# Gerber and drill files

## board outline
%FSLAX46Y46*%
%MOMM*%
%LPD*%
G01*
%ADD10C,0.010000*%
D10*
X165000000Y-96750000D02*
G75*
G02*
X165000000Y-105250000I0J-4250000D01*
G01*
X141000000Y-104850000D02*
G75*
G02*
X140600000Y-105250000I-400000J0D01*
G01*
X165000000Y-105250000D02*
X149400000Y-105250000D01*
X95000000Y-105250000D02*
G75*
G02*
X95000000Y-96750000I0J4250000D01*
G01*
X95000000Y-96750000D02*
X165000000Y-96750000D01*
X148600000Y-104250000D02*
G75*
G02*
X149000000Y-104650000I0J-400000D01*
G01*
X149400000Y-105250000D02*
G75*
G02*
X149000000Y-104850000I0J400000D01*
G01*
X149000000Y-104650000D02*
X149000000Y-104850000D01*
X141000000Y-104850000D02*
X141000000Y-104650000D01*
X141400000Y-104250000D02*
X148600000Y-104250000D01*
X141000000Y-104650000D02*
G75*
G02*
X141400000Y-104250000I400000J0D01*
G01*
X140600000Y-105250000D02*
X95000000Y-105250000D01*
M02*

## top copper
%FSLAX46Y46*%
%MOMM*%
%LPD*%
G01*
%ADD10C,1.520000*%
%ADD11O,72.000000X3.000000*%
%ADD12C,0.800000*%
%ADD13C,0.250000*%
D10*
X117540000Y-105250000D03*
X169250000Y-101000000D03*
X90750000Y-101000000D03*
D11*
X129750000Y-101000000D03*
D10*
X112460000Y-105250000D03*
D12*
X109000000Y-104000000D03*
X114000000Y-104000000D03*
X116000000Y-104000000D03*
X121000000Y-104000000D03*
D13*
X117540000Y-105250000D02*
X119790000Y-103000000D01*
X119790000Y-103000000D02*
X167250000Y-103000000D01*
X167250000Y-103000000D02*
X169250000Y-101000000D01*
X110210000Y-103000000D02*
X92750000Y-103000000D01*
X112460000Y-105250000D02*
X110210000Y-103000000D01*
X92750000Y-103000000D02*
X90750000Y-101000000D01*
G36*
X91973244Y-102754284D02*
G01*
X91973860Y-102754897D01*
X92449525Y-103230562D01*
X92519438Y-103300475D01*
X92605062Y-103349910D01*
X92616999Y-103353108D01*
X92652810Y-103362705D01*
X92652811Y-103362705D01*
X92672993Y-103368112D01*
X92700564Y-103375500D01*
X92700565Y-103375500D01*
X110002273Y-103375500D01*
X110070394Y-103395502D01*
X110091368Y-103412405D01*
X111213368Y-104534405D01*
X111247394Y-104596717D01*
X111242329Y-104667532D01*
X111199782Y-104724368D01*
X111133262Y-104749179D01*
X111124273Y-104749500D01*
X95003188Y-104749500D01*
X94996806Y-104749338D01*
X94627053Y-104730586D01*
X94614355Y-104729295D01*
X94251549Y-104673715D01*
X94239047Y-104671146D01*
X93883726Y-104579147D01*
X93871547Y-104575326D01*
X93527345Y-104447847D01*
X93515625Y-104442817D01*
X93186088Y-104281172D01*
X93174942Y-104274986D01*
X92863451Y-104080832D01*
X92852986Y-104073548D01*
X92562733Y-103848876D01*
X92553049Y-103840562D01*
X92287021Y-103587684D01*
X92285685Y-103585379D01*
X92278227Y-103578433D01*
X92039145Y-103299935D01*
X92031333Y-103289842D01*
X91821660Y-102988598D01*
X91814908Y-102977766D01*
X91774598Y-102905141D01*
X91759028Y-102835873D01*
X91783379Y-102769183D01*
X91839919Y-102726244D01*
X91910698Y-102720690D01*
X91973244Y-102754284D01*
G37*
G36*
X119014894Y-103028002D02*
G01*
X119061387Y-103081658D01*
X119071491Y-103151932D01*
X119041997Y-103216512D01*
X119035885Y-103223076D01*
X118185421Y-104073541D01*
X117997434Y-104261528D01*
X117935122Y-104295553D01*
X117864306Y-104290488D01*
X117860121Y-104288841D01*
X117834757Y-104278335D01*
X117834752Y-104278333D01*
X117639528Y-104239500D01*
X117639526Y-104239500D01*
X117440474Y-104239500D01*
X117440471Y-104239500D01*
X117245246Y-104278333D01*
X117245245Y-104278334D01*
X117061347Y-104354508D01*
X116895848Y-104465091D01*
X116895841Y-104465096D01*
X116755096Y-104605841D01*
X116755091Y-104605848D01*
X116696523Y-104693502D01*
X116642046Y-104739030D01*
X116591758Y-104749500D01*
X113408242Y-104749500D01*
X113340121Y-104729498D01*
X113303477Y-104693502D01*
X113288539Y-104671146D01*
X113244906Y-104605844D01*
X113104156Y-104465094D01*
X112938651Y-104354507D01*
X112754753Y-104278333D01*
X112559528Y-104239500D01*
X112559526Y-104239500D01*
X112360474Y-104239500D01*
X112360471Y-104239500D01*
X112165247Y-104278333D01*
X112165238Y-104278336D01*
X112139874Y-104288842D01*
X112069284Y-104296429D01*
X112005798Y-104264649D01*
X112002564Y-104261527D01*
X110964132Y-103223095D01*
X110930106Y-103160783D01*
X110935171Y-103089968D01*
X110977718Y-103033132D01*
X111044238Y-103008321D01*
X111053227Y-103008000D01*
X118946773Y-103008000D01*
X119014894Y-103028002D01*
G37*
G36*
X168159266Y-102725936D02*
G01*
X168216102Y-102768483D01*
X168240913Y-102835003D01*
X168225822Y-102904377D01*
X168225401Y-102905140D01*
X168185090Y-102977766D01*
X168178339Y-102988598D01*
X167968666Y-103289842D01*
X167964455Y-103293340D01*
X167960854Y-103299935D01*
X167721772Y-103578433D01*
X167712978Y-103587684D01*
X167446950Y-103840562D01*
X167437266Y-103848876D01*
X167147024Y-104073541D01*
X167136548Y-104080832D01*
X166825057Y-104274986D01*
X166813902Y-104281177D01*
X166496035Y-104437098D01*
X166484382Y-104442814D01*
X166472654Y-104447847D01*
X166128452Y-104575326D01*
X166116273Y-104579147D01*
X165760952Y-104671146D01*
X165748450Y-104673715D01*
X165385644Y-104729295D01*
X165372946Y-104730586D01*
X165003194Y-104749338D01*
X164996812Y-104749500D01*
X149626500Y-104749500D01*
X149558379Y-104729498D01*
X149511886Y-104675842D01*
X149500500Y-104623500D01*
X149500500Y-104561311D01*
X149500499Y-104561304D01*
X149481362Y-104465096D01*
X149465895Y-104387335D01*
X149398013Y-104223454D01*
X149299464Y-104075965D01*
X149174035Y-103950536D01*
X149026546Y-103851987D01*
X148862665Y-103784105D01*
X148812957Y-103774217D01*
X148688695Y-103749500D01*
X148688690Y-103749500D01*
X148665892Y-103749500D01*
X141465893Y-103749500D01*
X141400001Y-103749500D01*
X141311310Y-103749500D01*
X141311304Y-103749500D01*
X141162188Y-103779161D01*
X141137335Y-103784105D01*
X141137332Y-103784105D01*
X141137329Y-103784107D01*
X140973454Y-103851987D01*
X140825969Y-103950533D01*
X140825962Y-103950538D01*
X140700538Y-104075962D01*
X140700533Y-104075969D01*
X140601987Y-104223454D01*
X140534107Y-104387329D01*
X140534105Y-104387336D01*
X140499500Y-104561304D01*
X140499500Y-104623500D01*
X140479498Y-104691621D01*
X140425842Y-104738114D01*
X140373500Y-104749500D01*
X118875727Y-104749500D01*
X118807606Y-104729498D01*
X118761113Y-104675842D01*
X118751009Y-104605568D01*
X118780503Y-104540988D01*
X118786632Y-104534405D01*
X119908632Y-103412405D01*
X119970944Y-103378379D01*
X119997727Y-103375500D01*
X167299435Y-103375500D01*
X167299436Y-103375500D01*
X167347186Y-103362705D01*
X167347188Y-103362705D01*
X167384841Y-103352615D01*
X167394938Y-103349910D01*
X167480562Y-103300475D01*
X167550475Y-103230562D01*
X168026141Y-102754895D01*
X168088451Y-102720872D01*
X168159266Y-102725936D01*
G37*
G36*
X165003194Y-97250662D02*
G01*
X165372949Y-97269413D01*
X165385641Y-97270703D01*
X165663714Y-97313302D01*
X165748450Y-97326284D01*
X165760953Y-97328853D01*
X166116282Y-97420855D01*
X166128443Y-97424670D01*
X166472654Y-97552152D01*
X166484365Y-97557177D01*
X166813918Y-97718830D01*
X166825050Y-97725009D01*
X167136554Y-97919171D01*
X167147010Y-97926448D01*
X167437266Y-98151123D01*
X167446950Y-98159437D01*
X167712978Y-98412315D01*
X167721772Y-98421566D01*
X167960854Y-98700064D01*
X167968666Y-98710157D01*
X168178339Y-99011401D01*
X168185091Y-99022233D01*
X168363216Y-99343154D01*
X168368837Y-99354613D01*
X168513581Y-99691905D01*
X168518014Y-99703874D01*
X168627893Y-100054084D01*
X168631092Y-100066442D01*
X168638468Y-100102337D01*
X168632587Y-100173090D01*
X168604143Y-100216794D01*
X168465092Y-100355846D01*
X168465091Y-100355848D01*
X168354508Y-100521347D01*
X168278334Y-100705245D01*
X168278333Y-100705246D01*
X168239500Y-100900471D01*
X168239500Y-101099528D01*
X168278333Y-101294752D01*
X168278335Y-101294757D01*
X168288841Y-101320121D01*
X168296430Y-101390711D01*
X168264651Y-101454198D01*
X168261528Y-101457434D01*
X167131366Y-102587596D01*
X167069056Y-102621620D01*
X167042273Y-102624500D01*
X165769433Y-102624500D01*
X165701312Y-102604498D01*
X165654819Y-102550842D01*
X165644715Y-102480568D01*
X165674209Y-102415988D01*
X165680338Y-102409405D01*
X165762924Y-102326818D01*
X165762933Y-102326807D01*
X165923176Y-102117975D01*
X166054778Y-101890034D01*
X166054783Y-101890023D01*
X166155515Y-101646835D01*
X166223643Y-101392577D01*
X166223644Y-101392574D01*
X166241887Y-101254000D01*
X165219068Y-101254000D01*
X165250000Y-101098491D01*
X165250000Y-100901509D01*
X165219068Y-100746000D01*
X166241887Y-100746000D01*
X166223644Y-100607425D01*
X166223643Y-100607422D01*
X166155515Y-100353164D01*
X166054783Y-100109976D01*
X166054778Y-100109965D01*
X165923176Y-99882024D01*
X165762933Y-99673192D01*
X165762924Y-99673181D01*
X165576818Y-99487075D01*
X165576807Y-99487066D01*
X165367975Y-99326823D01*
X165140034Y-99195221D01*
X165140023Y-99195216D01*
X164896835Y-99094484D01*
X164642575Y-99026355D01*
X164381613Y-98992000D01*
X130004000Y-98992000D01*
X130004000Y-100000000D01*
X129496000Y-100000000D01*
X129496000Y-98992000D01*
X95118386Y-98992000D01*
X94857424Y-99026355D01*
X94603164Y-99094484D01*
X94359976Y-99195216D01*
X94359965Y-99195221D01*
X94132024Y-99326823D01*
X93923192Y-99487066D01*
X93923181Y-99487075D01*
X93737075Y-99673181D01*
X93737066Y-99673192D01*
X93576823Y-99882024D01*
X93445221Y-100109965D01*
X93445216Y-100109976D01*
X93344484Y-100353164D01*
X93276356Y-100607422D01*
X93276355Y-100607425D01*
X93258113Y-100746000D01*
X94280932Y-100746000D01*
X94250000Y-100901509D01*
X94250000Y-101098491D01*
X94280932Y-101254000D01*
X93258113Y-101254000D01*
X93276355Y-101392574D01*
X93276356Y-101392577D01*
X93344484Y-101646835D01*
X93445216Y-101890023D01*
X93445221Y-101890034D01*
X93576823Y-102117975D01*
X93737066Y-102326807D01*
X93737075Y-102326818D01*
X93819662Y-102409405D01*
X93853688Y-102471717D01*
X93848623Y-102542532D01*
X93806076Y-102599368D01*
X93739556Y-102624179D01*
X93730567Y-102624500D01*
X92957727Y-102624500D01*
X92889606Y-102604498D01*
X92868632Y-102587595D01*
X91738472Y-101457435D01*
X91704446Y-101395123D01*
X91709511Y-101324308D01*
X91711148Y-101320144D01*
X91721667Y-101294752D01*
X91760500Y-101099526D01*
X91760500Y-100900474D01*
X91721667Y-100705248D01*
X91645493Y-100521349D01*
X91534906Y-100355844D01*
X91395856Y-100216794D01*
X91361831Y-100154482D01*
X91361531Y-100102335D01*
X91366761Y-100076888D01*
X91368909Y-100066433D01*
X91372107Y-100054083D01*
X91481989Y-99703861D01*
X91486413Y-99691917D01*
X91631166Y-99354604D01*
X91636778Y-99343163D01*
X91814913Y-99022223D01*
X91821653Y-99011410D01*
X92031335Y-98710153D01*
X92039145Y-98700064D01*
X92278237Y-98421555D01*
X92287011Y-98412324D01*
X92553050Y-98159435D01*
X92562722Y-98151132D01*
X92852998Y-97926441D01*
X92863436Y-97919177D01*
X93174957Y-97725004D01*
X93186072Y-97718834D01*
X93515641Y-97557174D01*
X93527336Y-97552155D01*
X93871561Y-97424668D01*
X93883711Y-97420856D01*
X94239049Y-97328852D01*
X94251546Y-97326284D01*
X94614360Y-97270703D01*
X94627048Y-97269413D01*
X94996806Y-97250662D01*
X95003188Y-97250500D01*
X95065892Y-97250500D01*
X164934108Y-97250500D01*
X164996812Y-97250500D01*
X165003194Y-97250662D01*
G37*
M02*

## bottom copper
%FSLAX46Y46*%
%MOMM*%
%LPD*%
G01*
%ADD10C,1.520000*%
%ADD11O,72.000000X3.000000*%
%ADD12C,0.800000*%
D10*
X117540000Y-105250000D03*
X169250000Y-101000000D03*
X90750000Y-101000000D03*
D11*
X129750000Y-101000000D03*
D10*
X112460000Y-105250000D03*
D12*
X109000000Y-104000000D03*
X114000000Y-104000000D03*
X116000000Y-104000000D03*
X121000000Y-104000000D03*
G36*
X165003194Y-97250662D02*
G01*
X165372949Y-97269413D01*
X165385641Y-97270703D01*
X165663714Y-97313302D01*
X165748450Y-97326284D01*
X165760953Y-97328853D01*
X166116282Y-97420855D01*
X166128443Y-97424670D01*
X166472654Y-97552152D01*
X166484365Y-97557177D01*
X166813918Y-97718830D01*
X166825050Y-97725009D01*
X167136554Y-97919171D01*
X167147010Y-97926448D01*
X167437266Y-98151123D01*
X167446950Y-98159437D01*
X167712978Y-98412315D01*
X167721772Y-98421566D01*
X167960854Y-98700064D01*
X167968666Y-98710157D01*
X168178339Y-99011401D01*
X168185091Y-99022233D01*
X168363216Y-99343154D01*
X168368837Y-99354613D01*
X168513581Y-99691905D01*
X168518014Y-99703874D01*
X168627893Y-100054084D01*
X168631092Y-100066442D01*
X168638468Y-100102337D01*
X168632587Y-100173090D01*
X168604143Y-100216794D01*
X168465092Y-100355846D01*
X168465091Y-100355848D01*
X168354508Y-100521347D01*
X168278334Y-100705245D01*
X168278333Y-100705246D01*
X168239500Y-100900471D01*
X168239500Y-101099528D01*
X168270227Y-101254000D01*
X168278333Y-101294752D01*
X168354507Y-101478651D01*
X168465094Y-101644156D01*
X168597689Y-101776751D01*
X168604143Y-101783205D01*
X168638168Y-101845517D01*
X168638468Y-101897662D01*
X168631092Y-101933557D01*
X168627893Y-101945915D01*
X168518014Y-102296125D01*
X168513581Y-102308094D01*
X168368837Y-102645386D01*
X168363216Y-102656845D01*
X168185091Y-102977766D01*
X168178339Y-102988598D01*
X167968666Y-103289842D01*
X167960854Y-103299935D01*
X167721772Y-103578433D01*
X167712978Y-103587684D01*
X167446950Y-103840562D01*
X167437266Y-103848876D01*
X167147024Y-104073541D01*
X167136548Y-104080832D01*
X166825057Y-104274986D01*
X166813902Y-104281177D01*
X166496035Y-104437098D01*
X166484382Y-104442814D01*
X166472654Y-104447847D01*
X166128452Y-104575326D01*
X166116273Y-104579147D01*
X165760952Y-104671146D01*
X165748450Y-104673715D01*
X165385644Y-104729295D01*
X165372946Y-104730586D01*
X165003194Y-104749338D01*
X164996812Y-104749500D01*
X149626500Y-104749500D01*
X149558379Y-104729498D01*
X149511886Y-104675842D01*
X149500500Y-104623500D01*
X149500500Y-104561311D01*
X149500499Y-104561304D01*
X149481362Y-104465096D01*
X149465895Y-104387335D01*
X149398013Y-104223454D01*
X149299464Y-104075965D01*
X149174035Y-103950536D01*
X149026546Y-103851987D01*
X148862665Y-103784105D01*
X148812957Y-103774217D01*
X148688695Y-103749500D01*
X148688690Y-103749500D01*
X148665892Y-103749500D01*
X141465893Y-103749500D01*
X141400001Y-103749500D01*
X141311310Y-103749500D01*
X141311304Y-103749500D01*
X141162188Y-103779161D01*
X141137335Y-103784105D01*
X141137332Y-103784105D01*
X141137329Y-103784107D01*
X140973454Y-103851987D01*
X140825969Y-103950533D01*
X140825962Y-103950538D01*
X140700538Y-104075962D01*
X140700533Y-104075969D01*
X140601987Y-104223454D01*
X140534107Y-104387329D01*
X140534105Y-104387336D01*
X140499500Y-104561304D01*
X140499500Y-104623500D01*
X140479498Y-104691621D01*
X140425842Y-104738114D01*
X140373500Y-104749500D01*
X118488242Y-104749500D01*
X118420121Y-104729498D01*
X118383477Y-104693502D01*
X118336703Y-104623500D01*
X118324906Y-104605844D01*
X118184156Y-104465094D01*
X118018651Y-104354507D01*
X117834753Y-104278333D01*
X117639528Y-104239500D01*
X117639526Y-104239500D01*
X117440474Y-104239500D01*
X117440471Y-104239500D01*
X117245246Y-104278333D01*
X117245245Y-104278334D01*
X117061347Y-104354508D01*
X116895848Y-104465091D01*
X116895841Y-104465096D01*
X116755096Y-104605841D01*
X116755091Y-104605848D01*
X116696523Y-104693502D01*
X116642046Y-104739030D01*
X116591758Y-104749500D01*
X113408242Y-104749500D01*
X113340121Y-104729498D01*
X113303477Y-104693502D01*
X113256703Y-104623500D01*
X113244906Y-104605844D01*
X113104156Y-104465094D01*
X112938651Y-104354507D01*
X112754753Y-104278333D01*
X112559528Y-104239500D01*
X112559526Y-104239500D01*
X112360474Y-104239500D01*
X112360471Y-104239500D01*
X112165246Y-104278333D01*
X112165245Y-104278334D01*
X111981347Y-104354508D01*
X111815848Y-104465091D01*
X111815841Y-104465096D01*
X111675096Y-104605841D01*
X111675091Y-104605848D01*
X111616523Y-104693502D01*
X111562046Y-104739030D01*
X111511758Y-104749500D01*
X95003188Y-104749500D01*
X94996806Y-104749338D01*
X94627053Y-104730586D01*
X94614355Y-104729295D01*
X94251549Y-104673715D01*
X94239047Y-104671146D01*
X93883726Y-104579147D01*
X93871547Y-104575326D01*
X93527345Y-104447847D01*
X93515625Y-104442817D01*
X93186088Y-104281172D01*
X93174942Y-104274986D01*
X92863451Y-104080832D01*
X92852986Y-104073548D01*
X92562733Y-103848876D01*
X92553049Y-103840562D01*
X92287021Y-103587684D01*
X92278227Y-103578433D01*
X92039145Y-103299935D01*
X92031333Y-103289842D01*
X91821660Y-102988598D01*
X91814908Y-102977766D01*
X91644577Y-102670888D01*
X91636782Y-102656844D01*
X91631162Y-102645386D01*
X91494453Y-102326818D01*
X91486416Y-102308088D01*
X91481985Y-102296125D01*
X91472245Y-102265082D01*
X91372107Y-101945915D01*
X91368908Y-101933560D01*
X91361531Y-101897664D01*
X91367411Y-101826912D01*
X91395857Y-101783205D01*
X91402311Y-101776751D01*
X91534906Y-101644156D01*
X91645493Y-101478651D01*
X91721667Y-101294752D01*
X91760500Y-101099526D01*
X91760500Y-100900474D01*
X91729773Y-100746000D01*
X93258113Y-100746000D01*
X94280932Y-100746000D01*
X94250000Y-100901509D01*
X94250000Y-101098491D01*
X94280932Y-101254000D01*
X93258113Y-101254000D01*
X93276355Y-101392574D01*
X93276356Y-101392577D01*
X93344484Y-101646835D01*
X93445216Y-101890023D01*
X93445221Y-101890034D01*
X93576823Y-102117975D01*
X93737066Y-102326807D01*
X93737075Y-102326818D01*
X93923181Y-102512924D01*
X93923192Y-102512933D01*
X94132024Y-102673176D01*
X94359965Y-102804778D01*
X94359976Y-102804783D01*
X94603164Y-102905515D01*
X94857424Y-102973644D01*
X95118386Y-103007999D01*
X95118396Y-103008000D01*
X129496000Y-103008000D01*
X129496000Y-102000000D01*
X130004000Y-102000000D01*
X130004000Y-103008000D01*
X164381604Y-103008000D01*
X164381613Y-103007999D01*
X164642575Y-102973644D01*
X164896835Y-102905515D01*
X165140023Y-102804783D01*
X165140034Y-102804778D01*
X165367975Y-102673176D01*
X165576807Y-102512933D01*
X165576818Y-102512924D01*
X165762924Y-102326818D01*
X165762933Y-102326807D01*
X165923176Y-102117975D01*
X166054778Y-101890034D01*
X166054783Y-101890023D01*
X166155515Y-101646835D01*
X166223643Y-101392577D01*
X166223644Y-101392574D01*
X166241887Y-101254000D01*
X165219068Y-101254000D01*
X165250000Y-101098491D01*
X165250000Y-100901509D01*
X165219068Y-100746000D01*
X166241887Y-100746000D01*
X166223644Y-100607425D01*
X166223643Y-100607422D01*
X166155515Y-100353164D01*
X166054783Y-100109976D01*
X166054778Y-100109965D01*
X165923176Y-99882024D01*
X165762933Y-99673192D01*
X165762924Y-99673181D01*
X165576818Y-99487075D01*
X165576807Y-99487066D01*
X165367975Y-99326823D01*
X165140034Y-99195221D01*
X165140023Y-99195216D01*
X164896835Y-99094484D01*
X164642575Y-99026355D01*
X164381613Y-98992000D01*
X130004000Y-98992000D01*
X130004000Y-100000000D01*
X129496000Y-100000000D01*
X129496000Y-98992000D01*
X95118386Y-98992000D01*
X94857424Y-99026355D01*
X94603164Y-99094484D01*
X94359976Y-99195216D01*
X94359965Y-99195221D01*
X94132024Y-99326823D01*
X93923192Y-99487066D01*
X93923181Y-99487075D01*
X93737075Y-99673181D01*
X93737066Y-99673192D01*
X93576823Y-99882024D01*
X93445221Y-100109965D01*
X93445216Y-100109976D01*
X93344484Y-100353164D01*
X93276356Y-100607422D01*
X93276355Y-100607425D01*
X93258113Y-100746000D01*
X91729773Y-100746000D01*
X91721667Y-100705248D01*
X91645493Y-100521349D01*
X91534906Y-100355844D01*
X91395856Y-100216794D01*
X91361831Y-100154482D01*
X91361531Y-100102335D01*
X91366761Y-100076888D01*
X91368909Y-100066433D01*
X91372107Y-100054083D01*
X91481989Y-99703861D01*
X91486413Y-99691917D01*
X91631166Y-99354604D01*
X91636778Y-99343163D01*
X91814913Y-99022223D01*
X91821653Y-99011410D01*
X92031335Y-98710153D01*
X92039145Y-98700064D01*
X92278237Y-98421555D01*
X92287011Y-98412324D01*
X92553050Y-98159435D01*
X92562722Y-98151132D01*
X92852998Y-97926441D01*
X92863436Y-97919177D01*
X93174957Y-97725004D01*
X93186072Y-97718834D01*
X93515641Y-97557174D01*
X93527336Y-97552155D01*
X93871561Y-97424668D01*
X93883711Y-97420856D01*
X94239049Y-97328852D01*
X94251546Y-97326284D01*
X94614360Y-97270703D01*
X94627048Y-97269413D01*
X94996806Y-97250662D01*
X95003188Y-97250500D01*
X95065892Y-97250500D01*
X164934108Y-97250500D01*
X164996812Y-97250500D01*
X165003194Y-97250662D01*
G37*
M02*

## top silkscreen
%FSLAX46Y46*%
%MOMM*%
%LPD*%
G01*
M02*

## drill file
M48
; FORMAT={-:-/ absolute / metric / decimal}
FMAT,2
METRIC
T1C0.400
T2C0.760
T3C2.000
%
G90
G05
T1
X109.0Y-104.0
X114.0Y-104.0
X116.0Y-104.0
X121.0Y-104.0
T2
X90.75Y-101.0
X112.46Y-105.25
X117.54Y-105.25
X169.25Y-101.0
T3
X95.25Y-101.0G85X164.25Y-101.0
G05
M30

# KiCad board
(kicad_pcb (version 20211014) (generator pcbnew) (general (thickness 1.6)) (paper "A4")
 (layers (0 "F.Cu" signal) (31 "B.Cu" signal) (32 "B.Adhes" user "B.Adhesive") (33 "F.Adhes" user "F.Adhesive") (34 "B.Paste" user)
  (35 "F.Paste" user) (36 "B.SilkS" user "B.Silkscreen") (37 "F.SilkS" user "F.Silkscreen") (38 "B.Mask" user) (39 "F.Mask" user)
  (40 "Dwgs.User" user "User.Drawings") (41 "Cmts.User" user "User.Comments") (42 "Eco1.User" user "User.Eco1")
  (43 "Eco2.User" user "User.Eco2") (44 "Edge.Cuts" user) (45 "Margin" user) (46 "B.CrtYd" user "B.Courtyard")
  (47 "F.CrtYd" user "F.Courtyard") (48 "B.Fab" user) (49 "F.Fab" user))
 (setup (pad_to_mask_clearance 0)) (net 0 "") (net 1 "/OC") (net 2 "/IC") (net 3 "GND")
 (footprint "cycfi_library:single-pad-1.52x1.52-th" (layer "F.Cu") (at 117.54 105.25 180)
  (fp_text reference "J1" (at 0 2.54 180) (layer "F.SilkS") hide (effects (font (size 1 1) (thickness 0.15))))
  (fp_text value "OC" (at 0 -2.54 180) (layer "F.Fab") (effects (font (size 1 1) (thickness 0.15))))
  (pad "1" thru_hole circle (at 0 0 180) (size 1.52 1.52) (drill 0.76) (layers *.Cu *.Mask) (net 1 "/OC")))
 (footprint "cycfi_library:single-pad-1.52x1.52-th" (layer "F.Cu") (at 169.25 101 180)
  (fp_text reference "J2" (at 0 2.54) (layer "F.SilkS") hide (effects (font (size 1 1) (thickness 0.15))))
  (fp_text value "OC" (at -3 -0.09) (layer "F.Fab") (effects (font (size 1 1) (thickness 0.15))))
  (pad "1" thru_hole circle (at 0 0 180) (size 1.52 1.52) (drill 0.76) (layers *.Cu *.Mask) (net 1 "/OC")))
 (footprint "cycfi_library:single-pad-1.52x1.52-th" (layer "F.Cu") (at 90.75 101)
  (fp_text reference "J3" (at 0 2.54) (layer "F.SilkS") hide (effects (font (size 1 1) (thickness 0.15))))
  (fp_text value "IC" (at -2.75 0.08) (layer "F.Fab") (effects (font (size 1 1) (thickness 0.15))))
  (pad "1" thru_hole circle (at 0 0) (size 1.52 1.52) (drill 0.76) (layers *.Cu *.Mask) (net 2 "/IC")))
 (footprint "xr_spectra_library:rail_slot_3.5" (layer "F.Cu") (at 129.75 101)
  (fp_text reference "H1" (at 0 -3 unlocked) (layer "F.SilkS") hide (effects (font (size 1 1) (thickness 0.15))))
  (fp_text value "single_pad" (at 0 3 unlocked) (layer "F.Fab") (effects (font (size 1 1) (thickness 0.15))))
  (pad "1" thru_hole oval (at 0 0) (size 72 3) (drill oval 71 2) (layers *.Cu "B.Mask") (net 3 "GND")))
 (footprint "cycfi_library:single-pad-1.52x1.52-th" (layer "F.Cu") (at 112.46 105.25)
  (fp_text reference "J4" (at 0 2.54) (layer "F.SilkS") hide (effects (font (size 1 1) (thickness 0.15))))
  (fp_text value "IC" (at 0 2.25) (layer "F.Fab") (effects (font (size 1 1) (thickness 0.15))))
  (pad "1" thru_hole circle (at 0 0) (size 1.52 1.52) (drill 0.76) (layers *.Cu *.Mask) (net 2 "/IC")))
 (gr_arc (start 165 96.75) (mid 169.25 101) (end 165 105.25) (layer "Edge.Cuts") (width 0.01))
 (gr_arc (start 141 104.85) (mid 140.882843 105.132843) (end 140.6 105.25) (layer "Edge.Cuts") (width 0.01))
 (gr_line (start 165 105.25) (end 149.4 105.25) (layer "Edge.Cuts") (width 0.01))
 (gr_arc (start 95 105.25) (mid 90.75 101) (end 95 96.75) (layer "Edge.Cuts") (width 0.01))
 (gr_line (start 95 96.75) (end 165 96.75) (layer "Edge.Cuts") (width 0.01))
 (gr_arc (start 148.6 104.25) (mid 148.882843 104.367157) (end 149 104.65) (layer "Edge.Cuts") (width 0.01))
 (gr_arc (start 149.4 105.25) (mid 149.117157 105.132843) (end 149 104.85) (layer "Edge.Cuts") (width 0.01))
 (gr_line (start 149 104.65) (end 149 104.85) (layer "Edge.Cuts") (width 0.01))
 (gr_line (start 141 104.85) (end 141 104.65) (layer "Edge.Cuts") (width 0.01))
 (gr_line (start 141.4 104.25) (end 148.6 104.25) (layer "Edge.Cuts") (width 0.01))
 (gr_arc (start 141 104.65) (mid 141.117157 104.367157) (end 141.4 104.25) (layer "Edge.Cuts") (width 0.01))
 (gr_line (start 140.6 105.25) (end 95 105.25) (layer "Edge.Cuts") (width 0.01))
 (via (at 109 104) (size 0.8) (drill 0.4) (layers "F.Cu" "B.Cu") (free) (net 3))
 (via (at 114 104) (size 0.8) (drill 0.4) (layers "F.Cu" "B.Cu") (free) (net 3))
 (via (at 116 104) (size 0.8) (drill 0.4) (layers "F.Cu" "B.Cu") (free) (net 3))
 (via (at 121 104) (size 0.8) (drill 0.4) (layers "F.Cu" "B.Cu") (free) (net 3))
 (segment (start 117.54 105.25) (end 119.79 103) (width 0.25) (layer "F.Cu") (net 1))
 (segment (start 119.79 103) (end 167.25 103) (width 0.25) (layer "F.Cu") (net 1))
 (segment (start 167.25 103) (end 169.25 101) (width 0.25) (layer "F.Cu") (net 1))
 (segment (start 110.21 103) (end 92.75 103) (width 0.25) (layer "F.Cu") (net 2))
 (segment (start 112.46 105.25) (end 110.21 103) (width 0.25) (layer "F.Cu") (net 2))
 (segment (start 92.75 103) (end 90.75 101) (width 0.25) (layer "F.Cu") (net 2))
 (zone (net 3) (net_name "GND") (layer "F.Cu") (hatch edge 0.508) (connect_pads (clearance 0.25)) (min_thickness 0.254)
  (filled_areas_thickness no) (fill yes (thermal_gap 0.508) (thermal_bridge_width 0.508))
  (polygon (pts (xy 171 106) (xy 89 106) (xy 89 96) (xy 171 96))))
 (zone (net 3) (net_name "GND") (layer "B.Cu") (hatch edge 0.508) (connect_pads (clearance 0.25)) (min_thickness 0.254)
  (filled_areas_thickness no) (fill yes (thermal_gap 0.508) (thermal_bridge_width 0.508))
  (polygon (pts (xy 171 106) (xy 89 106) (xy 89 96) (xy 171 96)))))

